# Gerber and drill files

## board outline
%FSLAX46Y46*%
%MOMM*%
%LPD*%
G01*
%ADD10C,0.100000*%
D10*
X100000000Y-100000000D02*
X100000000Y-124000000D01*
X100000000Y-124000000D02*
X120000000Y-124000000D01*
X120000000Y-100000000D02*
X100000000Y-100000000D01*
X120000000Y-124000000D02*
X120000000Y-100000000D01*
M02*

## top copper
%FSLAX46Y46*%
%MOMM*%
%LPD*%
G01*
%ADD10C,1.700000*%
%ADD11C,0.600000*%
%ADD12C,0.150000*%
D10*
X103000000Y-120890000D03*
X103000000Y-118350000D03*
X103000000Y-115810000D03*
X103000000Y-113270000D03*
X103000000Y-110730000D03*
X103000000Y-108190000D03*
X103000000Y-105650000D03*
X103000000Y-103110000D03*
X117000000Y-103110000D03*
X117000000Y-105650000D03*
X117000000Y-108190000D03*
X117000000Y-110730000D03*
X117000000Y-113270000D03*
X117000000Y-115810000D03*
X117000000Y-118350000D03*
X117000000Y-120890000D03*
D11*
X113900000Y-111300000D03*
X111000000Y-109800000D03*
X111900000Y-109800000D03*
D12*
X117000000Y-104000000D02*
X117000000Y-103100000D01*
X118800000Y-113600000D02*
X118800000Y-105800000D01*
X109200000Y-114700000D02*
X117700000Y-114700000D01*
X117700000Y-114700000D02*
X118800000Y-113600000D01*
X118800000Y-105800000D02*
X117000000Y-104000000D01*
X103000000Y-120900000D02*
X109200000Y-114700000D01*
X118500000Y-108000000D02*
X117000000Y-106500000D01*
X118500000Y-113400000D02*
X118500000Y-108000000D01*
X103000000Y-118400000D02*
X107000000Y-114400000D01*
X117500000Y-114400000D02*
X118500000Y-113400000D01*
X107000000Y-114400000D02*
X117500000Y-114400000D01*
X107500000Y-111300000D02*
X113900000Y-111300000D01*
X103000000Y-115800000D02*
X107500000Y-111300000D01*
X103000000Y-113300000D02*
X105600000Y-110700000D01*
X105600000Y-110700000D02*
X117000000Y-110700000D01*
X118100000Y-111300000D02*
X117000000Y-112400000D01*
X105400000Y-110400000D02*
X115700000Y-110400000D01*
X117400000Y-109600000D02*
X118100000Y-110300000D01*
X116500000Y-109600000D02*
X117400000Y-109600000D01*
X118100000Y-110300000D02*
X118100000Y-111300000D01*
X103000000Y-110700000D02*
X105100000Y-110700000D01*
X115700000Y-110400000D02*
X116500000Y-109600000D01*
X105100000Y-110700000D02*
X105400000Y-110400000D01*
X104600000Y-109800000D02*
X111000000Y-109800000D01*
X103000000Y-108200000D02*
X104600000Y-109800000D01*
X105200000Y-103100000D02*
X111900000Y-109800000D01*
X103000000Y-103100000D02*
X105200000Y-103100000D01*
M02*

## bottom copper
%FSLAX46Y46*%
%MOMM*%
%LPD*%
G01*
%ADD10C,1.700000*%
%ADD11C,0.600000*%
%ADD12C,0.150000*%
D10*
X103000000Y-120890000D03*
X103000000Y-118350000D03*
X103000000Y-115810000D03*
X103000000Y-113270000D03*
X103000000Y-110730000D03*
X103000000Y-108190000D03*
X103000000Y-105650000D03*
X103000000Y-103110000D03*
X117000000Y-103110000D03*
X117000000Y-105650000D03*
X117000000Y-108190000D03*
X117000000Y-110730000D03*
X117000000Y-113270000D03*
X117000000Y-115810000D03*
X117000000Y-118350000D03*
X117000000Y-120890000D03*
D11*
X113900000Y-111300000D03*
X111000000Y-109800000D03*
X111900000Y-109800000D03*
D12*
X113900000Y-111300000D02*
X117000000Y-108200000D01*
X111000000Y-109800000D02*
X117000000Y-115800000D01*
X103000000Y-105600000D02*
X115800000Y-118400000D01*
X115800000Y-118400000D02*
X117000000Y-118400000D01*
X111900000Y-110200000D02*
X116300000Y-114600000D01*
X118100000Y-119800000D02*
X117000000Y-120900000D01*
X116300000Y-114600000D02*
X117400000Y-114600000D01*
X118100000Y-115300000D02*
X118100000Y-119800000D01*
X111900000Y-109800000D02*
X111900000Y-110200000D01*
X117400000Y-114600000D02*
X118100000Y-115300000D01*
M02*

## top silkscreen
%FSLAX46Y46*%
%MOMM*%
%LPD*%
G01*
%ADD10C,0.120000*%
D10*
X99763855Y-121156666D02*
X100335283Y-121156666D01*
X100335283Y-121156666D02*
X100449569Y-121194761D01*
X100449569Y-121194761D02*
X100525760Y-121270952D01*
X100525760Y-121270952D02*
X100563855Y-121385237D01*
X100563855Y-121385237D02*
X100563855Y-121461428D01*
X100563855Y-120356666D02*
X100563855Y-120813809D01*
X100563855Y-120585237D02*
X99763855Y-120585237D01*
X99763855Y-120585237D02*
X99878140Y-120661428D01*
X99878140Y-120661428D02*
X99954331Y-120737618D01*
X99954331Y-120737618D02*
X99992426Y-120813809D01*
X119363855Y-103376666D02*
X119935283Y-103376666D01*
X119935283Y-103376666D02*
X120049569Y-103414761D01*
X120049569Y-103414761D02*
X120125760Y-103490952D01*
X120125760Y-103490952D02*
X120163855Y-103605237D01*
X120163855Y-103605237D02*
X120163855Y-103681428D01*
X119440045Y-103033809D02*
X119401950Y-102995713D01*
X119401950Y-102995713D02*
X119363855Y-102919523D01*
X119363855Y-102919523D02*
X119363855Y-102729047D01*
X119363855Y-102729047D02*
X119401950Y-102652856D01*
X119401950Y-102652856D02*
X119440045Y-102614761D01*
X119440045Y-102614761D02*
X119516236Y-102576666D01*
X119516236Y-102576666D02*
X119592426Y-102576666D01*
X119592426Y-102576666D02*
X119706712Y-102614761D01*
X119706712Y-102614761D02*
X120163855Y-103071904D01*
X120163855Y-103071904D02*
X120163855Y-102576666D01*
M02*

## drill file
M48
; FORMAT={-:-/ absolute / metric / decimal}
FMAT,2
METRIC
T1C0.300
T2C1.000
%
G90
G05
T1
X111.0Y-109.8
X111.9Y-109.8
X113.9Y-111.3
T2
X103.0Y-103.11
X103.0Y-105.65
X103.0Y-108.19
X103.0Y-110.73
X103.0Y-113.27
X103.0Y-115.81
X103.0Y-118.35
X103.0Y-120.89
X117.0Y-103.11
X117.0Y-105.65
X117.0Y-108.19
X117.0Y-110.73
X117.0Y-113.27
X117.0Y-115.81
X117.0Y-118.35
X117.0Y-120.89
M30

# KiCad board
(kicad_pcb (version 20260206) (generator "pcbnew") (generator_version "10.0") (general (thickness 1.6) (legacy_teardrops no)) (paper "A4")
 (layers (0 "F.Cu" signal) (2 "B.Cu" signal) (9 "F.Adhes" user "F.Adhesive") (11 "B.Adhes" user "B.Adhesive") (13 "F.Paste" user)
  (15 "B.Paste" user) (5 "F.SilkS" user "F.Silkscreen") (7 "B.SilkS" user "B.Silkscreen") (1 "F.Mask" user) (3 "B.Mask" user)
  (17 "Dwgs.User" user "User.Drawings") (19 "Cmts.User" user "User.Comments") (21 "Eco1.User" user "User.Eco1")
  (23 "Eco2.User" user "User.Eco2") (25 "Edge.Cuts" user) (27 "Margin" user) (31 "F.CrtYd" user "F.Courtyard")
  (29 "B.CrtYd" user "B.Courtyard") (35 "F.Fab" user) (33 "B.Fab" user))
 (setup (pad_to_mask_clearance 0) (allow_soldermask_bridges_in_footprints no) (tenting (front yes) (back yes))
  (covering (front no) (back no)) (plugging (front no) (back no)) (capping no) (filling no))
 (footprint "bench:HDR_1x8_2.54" (layer "F.Cu") (at 103 120.89 90)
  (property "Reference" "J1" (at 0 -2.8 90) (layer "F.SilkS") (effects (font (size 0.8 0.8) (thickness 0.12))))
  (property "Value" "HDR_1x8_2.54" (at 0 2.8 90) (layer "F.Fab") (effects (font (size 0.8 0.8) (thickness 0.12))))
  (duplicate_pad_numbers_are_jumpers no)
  (pad "1" thru_hole circle (at 0 0 90) (size 1.7 1.7) (drill 1) (layers "*.Cu" "*.Mask") (remove_unused_layers no) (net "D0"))
  (pad "2" thru_hole circle (at 2.54 0 90) (size 1.7 1.7) (drill 1) (layers "*.Cu" "*.Mask") (remove_unused_layers no) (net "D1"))
  (pad "3" thru_hole circle (at 5.08 0 90) (size 1.7 1.7) (drill 1) (layers "*.Cu" "*.Mask") (remove_unused_layers no) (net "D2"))
  (pad "4" thru_hole circle (at 7.62 0 90) (size 1.7 1.7) (drill 1) (layers "*.Cu" "*.Mask") (remove_unused_layers no) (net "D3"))
  (pad "5" thru_hole circle (at 10.16 0 90) (size 1.7 1.7) (drill 1) (layers "*.Cu" "*.Mask") (remove_unused_layers no) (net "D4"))
  (pad "6" thru_hole circle (at 12.7 0 90) (size 1.7 1.7) (drill 1) (layers "*.Cu" "*.Mask") (remove_unused_layers no) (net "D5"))
  (pad "7" thru_hole circle (at 15.24 0 90) (size 1.7 1.7) (drill 1) (layers "*.Cu" "*.Mask") (remove_unused_layers no) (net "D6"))
  (pad "8" thru_hole circle (at 17.78 0 90) (size 1.7 1.7) (drill 1) (layers "*.Cu" "*.Mask") (remove_unused_layers no) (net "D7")))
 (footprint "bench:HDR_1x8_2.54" (layer "F.Cu") (at 117 103.11 -90)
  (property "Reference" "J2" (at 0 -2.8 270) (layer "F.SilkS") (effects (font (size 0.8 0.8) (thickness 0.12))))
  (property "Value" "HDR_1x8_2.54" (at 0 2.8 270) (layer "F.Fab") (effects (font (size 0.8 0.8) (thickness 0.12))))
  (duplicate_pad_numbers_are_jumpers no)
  (pad "1" thru_hole circle (at 0 0 270) (size 1.7 1.7) (drill 1) (layers "*.Cu" "*.Mask") (remove_unused_layers no) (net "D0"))
  (pad "2" thru_hole circle (at 2.54 0 270) (size 1.7 1.7) (drill 1) (layers "*.Cu" "*.Mask") (remove_unused_layers no) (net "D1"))
  (pad "3" thru_hole circle (at 5.08 0 270) (size 1.7 1.7) (drill 1) (layers "*.Cu" "*.Mask") (remove_unused_layers no) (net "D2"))
  (pad "4" thru_hole circle (at 7.62 0 270) (size 1.7 1.7) (drill 1) (layers "*.Cu" "*.Mask") (remove_unused_layers no) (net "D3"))
  (pad "5" thru_hole circle (at 10.16 0 270) (size 1.7 1.7) (drill 1) (layers "*.Cu" "*.Mask") (remove_unused_layers no) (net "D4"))
  (pad "6" thru_hole circle (at 12.7 0 270) (size 1.7 1.7) (drill 1) (layers "*.Cu" "*.Mask") (remove_unused_layers no) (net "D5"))
  (pad "7" thru_hole circle (at 15.24 0 270) (size 1.7 1.7) (drill 1) (layers "*.Cu" "*.Mask") (remove_unused_layers no) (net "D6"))
  (pad "8" thru_hole circle (at 17.78 0 270) (size 1.7 1.7) (drill 1) (layers "*.Cu" "*.Mask") (remove_unused_layers no) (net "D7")))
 (gr_line (start 100 100) (end 100 124) (stroke (width 0.1) (type solid)) (layer "Edge.Cuts"))
 (gr_line (start 100 124) (end 120 124) (stroke (width 0.1) (type solid)) (layer "Edge.Cuts"))
 (gr_line (start 120 100) (end 100 100) (stroke (width 0.1) (type solid)) (layer "Edge.Cuts"))
 (gr_line (start 120 124) (end 120 100) (stroke (width 0.1) (type solid)) (layer "Edge.Cuts"))
 (segment (start 117 104) (end 117 103.1) (width 0.15) (layer "F.Cu") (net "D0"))
 (segment (start 118.8 113.6) (end 118.8 105.8) (width 0.15) (layer "F.Cu") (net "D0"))
 (segment (start 109.2 114.7) (end 117.7 114.7) (width 0.15) (layer "F.Cu") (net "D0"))
 (segment (start 117.7 114.7) (end 118.8 113.6) (width 0.15) (layer "F.Cu") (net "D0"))
 (segment (start 118.8 105.8) (end 117 104) (width 0.15) (layer "F.Cu") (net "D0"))
 (segment (start 103 120.9) (end 109.2 114.7) (width 0.15) (layer "F.Cu") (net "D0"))
 (segment (start 118.5 108) (end 117 106.5) (width 0.15) (layer "F.Cu") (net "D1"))
 (segment (start 118.5 113.4) (end 118.5 108) (width 0.15) (layer "F.Cu") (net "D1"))
 (segment (start 103 118.4) (end 107 114.4) (width 0.15) (layer "F.Cu") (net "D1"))
 (segment (start 117.5 114.4) (end 118.5 113.4) (width 0.15) (layer "F.Cu") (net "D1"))
 (segment (start 107 114.4) (end 117.5 114.4) (width 0.15) (layer "F.Cu") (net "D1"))
 (segment (start 107.5 111.3) (end 113.9 111.3) (width 0.15) (layer "F.Cu") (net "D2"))
 (segment (start 103 115.8) (end 107.5 111.3) (width 0.15) (layer "F.Cu") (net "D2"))
 (via (at 113.9 111.3) (size 0.6) (drill 0.3) (layers "F.Cu" "B.Cu") (capping no) (covering (front no) (back no))
  (plugging (front no) (back no)) (filling no) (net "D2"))
 (segment (start 113.9 111.3) (end 117 108.2) (width 0.15) (layer "B.Cu") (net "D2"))
 (segment (start 103 113.3) (end 105.6 110.7) (width 0.15) (layer "F.Cu") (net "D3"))
 (segment (start 105.6 110.7) (end 117 110.7) (width 0.15) (layer "F.Cu") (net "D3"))
 (segment (start 118.1 111.3) (end 117 112.4) (width 0.15) (layer "F.Cu") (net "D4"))
 (segment (start 105.4 110.4) (end 115.7 110.4) (width 0.15) (layer "F.Cu") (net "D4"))
 (segment (start 117.4 109.6) (end 118.1 110.3) (width 0.15) (layer "F.Cu") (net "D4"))
 (segment (start 116.5 109.6) (end 117.4 109.6) (width 0.15) (layer "F.Cu") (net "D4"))
 (segment (start 118.1 110.3) (end 118.1 111.3) (width 0.15) (layer "F.Cu") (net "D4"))
 (segment (start 103 110.7) (end 105.1 110.7) (width 0.15) (layer "F.Cu") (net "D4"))
 (segment (start 115.7 110.4) (end 116.5 109.6) (width 0.15) (layer "F.Cu") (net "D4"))
 (segment (start 105.1 110.7) (end 105.4 110.4) (width 0.15) (layer "F.Cu") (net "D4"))
 (segment (start 104.6 109.8) (end 111 109.8) (width 0.15) (layer "F.Cu") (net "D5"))
 (segment (start 103 108.2) (end 104.6 109.8) (width 0.15) (layer "F.Cu") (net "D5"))
 (via (at 111 109.8) (size 0.6) (drill 0.3) (layers "F.Cu" "B.Cu") (capping no) (covering (front no) (back no))
  (plugging (front no) (back no)) (filling no) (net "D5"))
 (segment (start 111 109.8) (end 117 115.8) (width 0.15) (layer "B.Cu") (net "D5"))
 (segment (start 103 105.6) (end 115.8 118.4) (width 0.15) (layer "B.Cu") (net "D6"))
 (segment (start 115.8 118.4) (end 117 118.4) (width 0.15) (layer "B.Cu") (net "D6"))
 (segment (start 105.2 103.1) (end 111.9 109.8) (width 0.15) (layer "F.Cu") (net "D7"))
 (segment (start 103 103.1) (end 105.2 103.1) (width 0.15) (layer "F.Cu") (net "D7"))
 (via (at 111.9 109.8) (size 0.6) (drill 0.3) (layers "F.Cu" "B.Cu") (capping no) (covering (front no) (back no))
  (plugging (front no) (back no)) (filling no) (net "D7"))
 (segment (start 111.9 110.2) (end 116.3 114.6) (width 0.15) (layer "B.Cu") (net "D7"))
 (segment (start 118.1 119.8) (end 117 120.9) (width 0.15) (layer "B.Cu") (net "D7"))
 (segment (start 116.3 114.6) (end 117.4 114.6) (width 0.15) (layer "B.Cu") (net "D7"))
 (segment (start 118.1 115.3) (end 118.1 119.8) (width 0.15) (layer "B.Cu") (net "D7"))
 (segment (start 111.9 109.8) (end 111.9 110.2) (width 0.15) (layer "B.Cu") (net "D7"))
 (segment (start 117.4 114.6) (end 118.1 115.3) (width 0.15) (layer "B.Cu") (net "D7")))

